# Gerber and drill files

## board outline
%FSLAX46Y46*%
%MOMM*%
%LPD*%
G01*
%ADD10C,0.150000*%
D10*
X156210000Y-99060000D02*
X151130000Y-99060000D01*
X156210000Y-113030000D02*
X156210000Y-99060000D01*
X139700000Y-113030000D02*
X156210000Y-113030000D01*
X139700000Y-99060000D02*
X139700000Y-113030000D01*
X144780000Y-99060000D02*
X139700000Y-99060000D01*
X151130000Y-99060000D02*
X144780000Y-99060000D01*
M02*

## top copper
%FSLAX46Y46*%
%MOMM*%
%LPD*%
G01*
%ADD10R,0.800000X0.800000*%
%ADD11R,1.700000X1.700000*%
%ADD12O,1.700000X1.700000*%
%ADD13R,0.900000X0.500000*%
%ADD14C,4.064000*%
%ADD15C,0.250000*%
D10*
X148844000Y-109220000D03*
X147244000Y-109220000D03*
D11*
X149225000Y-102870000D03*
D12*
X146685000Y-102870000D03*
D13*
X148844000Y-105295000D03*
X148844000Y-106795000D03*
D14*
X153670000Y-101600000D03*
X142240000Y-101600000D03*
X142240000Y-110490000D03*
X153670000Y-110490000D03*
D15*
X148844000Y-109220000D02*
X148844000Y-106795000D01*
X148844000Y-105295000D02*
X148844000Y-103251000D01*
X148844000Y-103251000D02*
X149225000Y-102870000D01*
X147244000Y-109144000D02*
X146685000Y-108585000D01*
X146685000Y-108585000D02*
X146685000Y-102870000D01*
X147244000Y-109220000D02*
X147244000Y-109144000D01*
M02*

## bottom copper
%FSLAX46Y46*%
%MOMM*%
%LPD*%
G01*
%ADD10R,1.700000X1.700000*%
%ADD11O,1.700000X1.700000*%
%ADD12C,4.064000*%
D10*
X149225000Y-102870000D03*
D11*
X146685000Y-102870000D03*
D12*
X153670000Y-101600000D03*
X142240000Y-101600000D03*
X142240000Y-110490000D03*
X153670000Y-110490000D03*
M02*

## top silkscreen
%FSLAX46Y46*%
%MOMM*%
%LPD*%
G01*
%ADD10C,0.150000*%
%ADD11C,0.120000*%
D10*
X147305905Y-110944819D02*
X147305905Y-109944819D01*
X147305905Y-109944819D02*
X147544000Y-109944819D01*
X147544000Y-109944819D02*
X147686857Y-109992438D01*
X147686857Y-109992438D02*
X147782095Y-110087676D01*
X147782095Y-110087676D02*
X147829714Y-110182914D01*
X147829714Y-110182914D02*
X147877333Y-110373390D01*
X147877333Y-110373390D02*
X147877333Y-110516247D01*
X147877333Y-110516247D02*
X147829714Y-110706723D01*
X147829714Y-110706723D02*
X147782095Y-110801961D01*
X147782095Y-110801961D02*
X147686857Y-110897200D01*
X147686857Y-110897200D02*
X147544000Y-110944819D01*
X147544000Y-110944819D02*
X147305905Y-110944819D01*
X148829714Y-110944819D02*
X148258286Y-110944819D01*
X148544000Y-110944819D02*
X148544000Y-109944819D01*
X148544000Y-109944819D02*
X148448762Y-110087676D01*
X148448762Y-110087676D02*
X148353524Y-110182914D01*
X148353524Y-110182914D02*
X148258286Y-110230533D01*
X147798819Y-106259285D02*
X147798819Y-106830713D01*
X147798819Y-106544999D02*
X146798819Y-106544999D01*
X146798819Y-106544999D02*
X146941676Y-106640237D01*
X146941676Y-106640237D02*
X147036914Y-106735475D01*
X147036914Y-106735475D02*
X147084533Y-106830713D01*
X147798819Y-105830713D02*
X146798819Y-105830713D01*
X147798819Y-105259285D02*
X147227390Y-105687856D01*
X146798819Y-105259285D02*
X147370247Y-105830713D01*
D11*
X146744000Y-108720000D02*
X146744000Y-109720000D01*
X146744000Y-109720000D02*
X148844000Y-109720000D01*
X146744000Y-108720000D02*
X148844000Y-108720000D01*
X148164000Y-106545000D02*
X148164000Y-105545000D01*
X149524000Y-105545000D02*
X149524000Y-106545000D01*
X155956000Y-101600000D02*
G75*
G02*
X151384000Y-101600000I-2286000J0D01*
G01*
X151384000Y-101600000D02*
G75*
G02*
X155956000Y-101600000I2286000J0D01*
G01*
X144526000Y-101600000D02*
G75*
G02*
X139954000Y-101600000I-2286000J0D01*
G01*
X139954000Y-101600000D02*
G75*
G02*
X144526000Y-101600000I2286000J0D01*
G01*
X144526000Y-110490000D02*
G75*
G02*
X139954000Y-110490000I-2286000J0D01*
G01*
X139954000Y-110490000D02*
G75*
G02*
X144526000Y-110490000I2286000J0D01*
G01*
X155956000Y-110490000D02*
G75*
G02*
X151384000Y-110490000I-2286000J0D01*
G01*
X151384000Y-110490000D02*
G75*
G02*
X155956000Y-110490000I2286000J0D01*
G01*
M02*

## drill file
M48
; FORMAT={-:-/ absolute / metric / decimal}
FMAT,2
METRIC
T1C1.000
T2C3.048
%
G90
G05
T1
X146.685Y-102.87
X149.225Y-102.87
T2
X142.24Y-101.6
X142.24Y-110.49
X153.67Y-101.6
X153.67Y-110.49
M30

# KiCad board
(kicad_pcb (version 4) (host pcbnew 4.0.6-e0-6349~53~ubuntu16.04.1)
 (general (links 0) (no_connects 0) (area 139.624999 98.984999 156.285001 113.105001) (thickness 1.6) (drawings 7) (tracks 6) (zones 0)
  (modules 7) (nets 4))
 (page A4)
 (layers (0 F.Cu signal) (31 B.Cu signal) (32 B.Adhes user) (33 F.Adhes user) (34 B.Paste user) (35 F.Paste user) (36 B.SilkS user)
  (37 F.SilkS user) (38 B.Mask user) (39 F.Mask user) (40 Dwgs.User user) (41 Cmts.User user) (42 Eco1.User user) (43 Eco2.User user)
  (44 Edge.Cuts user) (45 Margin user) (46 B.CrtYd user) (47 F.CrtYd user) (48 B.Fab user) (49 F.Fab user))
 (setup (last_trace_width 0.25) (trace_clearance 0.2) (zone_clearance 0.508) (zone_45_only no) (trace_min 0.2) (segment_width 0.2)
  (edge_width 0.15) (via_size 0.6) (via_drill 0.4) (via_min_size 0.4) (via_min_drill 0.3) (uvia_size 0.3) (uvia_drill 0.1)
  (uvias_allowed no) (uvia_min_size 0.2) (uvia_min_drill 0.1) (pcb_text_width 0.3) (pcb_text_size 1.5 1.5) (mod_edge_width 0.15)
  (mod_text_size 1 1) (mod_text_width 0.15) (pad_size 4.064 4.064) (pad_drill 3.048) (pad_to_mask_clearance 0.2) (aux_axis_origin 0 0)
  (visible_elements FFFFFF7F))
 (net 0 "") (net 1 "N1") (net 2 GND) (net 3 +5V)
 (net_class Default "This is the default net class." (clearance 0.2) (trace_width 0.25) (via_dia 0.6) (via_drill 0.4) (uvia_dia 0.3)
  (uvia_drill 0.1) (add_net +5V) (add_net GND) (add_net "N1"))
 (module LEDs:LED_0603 (layer F.Cu) (at 148.044 109.22)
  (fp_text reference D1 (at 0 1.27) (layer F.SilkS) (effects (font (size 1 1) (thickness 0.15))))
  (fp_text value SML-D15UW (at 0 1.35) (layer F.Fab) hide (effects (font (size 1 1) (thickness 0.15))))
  (fp_line (start -1.3 -0.5) (end -1.3 0.5) (layer F.SilkS) (width 0.12))
  (fp_line (start -1.3 0.5) (end 0.8 0.5) (layer F.SilkS) (width 0.12))
  (fp_line (start -1.3 -0.5) (end 0.8 -0.5) (layer F.SilkS) (width 0.12))
  (pad 2 smd rect (at 0.8 0 180) (size 0.8 0.8) (layers F.Cu F.Paste F.Mask) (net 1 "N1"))
  (pad 1 smd rect (at -0.8 0 180) (size 0.8 0.8) (layers F.Cu F.Paste F.Mask) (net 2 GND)))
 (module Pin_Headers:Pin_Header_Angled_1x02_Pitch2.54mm (layer B.Cu) (at 149.225 102.87 90)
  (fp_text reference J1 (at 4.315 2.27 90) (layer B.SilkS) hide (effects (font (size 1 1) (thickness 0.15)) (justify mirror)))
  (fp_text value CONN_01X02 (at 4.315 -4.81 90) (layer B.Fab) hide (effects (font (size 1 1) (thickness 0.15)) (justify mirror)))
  (pad 1 thru_hole rect (at 0 0 90) (size 1.7 1.7) (drill 1) (layers *.Cu *.Mask) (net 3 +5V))
  (pad 2 thru_hole oval (at 0 -2.54 90) (size 1.7 1.7) (drill 1) (layers *.Cu *.Mask) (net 2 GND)))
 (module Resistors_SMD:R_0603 (layer F.Cu) (at 148.844 106.045 270)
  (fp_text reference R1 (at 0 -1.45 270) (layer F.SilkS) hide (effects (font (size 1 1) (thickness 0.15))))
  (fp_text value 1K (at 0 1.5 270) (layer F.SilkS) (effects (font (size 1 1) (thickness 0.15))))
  (fp_line (start 0.5 0.68) (end -0.5 0.68) (layer F.SilkS) (width 0.12))
  (fp_line (start -0.5 -0.68) (end 0.5 -0.68) (layer F.SilkS) (width 0.12))
  (pad 1 smd rect (at -0.75 0 270) (size 0.5 0.9) (layers F.Cu F.Paste F.Mask) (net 3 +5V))
  (pad 2 smd rect (at 0.75 0 270) (size 0.5 0.9) (layers F.Cu F.Paste F.Mask) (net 1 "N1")))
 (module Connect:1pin (layer F.Cu) (at 153.67 101.6)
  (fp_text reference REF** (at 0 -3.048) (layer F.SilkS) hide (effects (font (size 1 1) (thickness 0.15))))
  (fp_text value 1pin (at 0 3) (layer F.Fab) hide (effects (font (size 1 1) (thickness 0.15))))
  (fp_circle (center 0 0) (end 0 -2.286) (layer F.SilkS) (width 0.12))
  (pad "" np_thru_hole circle (at 0 0) (size 4.064 4.064) (drill 3.048) (layers *.Cu *.Mask)))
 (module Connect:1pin (layer F.Cu) (at 142.24 101.6)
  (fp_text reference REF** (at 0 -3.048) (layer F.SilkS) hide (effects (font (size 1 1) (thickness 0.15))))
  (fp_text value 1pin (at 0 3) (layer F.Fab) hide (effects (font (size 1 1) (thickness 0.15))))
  (fp_circle (center 0 0) (end 0 -2.286) (layer F.SilkS) (width 0.12))
  (pad "" np_thru_hole circle (at 0 0) (size 4.064 4.064) (drill 3.048) (layers *.Cu *.Mask)))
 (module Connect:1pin (layer F.Cu) (at 142.24 110.49)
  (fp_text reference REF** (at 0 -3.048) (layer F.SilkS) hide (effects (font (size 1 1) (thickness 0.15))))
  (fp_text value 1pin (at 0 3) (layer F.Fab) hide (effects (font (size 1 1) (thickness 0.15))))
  (fp_circle (center 0 0) (end 0 -2.286) (layer F.SilkS) (width 0.12))
  (pad "" np_thru_hole circle (at 0 0) (size 4.064 4.064) (drill 3.048) (layers *.Cu *.Mask)))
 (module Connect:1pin (layer F.Cu) (at 153.67 110.49)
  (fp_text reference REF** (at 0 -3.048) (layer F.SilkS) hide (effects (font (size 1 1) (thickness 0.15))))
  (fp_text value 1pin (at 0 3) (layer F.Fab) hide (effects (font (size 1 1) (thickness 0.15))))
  (fp_circle (center 0 0) (end 0 -2.286) (layer F.SilkS) (width 0.12))
  (pad "" np_thru_hole circle (at 0 0) (size 4.064 4.064) (drill 3.048) (layers *.Cu *.Mask)))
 (gr_line (start 156.21 99.06) (end 151.13 99.06) (layer Edge.Cuts) (width 0.15))
 (gr_line (start 156.21 113.03) (end 156.21 99.06) (layer Edge.Cuts) (width 0.15))
 (gr_line (start 139.7 113.03) (end 156.21 113.03) (layer Edge.Cuts) (width 0.15))
 (gr_line (start 139.7 99.06) (end 139.7 113.03) (layer Edge.Cuts) (width 0.15))
 (gr_line (start 144.78 99.06) (end 139.7 99.06) (layer Edge.Cuts) (width 0.15))
 (gr_line (start 151.13 99.06) (end 144.78 99.06) (layer Edge.Cuts) (width 0.15))
 (segment (start 148.844 109.22) (end 148.844 106.795) (width 0.25) (layer F.Cu) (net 1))
 (segment (start 148.844 105.295) (end 148.844 103.251) (width 0.25) (layer F.Cu) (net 3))
 (segment (start 148.844 103.251) (end 149.225 102.87) (width 0.25) (layer F.Cu) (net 3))
 (segment (start 147.244 109.144) (end 146.685 108.585) (width 0.25) (layer F.Cu) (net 2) (status 10))
 (segment (start 146.685 108.585) (end 146.685 102.87) (width 0.25) (layer F.Cu) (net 2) (status 20))
 (segment (start 147.244 109.22) (end 147.244 109.144) (width 0.25) (layer F.Cu) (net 2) (status 30)))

